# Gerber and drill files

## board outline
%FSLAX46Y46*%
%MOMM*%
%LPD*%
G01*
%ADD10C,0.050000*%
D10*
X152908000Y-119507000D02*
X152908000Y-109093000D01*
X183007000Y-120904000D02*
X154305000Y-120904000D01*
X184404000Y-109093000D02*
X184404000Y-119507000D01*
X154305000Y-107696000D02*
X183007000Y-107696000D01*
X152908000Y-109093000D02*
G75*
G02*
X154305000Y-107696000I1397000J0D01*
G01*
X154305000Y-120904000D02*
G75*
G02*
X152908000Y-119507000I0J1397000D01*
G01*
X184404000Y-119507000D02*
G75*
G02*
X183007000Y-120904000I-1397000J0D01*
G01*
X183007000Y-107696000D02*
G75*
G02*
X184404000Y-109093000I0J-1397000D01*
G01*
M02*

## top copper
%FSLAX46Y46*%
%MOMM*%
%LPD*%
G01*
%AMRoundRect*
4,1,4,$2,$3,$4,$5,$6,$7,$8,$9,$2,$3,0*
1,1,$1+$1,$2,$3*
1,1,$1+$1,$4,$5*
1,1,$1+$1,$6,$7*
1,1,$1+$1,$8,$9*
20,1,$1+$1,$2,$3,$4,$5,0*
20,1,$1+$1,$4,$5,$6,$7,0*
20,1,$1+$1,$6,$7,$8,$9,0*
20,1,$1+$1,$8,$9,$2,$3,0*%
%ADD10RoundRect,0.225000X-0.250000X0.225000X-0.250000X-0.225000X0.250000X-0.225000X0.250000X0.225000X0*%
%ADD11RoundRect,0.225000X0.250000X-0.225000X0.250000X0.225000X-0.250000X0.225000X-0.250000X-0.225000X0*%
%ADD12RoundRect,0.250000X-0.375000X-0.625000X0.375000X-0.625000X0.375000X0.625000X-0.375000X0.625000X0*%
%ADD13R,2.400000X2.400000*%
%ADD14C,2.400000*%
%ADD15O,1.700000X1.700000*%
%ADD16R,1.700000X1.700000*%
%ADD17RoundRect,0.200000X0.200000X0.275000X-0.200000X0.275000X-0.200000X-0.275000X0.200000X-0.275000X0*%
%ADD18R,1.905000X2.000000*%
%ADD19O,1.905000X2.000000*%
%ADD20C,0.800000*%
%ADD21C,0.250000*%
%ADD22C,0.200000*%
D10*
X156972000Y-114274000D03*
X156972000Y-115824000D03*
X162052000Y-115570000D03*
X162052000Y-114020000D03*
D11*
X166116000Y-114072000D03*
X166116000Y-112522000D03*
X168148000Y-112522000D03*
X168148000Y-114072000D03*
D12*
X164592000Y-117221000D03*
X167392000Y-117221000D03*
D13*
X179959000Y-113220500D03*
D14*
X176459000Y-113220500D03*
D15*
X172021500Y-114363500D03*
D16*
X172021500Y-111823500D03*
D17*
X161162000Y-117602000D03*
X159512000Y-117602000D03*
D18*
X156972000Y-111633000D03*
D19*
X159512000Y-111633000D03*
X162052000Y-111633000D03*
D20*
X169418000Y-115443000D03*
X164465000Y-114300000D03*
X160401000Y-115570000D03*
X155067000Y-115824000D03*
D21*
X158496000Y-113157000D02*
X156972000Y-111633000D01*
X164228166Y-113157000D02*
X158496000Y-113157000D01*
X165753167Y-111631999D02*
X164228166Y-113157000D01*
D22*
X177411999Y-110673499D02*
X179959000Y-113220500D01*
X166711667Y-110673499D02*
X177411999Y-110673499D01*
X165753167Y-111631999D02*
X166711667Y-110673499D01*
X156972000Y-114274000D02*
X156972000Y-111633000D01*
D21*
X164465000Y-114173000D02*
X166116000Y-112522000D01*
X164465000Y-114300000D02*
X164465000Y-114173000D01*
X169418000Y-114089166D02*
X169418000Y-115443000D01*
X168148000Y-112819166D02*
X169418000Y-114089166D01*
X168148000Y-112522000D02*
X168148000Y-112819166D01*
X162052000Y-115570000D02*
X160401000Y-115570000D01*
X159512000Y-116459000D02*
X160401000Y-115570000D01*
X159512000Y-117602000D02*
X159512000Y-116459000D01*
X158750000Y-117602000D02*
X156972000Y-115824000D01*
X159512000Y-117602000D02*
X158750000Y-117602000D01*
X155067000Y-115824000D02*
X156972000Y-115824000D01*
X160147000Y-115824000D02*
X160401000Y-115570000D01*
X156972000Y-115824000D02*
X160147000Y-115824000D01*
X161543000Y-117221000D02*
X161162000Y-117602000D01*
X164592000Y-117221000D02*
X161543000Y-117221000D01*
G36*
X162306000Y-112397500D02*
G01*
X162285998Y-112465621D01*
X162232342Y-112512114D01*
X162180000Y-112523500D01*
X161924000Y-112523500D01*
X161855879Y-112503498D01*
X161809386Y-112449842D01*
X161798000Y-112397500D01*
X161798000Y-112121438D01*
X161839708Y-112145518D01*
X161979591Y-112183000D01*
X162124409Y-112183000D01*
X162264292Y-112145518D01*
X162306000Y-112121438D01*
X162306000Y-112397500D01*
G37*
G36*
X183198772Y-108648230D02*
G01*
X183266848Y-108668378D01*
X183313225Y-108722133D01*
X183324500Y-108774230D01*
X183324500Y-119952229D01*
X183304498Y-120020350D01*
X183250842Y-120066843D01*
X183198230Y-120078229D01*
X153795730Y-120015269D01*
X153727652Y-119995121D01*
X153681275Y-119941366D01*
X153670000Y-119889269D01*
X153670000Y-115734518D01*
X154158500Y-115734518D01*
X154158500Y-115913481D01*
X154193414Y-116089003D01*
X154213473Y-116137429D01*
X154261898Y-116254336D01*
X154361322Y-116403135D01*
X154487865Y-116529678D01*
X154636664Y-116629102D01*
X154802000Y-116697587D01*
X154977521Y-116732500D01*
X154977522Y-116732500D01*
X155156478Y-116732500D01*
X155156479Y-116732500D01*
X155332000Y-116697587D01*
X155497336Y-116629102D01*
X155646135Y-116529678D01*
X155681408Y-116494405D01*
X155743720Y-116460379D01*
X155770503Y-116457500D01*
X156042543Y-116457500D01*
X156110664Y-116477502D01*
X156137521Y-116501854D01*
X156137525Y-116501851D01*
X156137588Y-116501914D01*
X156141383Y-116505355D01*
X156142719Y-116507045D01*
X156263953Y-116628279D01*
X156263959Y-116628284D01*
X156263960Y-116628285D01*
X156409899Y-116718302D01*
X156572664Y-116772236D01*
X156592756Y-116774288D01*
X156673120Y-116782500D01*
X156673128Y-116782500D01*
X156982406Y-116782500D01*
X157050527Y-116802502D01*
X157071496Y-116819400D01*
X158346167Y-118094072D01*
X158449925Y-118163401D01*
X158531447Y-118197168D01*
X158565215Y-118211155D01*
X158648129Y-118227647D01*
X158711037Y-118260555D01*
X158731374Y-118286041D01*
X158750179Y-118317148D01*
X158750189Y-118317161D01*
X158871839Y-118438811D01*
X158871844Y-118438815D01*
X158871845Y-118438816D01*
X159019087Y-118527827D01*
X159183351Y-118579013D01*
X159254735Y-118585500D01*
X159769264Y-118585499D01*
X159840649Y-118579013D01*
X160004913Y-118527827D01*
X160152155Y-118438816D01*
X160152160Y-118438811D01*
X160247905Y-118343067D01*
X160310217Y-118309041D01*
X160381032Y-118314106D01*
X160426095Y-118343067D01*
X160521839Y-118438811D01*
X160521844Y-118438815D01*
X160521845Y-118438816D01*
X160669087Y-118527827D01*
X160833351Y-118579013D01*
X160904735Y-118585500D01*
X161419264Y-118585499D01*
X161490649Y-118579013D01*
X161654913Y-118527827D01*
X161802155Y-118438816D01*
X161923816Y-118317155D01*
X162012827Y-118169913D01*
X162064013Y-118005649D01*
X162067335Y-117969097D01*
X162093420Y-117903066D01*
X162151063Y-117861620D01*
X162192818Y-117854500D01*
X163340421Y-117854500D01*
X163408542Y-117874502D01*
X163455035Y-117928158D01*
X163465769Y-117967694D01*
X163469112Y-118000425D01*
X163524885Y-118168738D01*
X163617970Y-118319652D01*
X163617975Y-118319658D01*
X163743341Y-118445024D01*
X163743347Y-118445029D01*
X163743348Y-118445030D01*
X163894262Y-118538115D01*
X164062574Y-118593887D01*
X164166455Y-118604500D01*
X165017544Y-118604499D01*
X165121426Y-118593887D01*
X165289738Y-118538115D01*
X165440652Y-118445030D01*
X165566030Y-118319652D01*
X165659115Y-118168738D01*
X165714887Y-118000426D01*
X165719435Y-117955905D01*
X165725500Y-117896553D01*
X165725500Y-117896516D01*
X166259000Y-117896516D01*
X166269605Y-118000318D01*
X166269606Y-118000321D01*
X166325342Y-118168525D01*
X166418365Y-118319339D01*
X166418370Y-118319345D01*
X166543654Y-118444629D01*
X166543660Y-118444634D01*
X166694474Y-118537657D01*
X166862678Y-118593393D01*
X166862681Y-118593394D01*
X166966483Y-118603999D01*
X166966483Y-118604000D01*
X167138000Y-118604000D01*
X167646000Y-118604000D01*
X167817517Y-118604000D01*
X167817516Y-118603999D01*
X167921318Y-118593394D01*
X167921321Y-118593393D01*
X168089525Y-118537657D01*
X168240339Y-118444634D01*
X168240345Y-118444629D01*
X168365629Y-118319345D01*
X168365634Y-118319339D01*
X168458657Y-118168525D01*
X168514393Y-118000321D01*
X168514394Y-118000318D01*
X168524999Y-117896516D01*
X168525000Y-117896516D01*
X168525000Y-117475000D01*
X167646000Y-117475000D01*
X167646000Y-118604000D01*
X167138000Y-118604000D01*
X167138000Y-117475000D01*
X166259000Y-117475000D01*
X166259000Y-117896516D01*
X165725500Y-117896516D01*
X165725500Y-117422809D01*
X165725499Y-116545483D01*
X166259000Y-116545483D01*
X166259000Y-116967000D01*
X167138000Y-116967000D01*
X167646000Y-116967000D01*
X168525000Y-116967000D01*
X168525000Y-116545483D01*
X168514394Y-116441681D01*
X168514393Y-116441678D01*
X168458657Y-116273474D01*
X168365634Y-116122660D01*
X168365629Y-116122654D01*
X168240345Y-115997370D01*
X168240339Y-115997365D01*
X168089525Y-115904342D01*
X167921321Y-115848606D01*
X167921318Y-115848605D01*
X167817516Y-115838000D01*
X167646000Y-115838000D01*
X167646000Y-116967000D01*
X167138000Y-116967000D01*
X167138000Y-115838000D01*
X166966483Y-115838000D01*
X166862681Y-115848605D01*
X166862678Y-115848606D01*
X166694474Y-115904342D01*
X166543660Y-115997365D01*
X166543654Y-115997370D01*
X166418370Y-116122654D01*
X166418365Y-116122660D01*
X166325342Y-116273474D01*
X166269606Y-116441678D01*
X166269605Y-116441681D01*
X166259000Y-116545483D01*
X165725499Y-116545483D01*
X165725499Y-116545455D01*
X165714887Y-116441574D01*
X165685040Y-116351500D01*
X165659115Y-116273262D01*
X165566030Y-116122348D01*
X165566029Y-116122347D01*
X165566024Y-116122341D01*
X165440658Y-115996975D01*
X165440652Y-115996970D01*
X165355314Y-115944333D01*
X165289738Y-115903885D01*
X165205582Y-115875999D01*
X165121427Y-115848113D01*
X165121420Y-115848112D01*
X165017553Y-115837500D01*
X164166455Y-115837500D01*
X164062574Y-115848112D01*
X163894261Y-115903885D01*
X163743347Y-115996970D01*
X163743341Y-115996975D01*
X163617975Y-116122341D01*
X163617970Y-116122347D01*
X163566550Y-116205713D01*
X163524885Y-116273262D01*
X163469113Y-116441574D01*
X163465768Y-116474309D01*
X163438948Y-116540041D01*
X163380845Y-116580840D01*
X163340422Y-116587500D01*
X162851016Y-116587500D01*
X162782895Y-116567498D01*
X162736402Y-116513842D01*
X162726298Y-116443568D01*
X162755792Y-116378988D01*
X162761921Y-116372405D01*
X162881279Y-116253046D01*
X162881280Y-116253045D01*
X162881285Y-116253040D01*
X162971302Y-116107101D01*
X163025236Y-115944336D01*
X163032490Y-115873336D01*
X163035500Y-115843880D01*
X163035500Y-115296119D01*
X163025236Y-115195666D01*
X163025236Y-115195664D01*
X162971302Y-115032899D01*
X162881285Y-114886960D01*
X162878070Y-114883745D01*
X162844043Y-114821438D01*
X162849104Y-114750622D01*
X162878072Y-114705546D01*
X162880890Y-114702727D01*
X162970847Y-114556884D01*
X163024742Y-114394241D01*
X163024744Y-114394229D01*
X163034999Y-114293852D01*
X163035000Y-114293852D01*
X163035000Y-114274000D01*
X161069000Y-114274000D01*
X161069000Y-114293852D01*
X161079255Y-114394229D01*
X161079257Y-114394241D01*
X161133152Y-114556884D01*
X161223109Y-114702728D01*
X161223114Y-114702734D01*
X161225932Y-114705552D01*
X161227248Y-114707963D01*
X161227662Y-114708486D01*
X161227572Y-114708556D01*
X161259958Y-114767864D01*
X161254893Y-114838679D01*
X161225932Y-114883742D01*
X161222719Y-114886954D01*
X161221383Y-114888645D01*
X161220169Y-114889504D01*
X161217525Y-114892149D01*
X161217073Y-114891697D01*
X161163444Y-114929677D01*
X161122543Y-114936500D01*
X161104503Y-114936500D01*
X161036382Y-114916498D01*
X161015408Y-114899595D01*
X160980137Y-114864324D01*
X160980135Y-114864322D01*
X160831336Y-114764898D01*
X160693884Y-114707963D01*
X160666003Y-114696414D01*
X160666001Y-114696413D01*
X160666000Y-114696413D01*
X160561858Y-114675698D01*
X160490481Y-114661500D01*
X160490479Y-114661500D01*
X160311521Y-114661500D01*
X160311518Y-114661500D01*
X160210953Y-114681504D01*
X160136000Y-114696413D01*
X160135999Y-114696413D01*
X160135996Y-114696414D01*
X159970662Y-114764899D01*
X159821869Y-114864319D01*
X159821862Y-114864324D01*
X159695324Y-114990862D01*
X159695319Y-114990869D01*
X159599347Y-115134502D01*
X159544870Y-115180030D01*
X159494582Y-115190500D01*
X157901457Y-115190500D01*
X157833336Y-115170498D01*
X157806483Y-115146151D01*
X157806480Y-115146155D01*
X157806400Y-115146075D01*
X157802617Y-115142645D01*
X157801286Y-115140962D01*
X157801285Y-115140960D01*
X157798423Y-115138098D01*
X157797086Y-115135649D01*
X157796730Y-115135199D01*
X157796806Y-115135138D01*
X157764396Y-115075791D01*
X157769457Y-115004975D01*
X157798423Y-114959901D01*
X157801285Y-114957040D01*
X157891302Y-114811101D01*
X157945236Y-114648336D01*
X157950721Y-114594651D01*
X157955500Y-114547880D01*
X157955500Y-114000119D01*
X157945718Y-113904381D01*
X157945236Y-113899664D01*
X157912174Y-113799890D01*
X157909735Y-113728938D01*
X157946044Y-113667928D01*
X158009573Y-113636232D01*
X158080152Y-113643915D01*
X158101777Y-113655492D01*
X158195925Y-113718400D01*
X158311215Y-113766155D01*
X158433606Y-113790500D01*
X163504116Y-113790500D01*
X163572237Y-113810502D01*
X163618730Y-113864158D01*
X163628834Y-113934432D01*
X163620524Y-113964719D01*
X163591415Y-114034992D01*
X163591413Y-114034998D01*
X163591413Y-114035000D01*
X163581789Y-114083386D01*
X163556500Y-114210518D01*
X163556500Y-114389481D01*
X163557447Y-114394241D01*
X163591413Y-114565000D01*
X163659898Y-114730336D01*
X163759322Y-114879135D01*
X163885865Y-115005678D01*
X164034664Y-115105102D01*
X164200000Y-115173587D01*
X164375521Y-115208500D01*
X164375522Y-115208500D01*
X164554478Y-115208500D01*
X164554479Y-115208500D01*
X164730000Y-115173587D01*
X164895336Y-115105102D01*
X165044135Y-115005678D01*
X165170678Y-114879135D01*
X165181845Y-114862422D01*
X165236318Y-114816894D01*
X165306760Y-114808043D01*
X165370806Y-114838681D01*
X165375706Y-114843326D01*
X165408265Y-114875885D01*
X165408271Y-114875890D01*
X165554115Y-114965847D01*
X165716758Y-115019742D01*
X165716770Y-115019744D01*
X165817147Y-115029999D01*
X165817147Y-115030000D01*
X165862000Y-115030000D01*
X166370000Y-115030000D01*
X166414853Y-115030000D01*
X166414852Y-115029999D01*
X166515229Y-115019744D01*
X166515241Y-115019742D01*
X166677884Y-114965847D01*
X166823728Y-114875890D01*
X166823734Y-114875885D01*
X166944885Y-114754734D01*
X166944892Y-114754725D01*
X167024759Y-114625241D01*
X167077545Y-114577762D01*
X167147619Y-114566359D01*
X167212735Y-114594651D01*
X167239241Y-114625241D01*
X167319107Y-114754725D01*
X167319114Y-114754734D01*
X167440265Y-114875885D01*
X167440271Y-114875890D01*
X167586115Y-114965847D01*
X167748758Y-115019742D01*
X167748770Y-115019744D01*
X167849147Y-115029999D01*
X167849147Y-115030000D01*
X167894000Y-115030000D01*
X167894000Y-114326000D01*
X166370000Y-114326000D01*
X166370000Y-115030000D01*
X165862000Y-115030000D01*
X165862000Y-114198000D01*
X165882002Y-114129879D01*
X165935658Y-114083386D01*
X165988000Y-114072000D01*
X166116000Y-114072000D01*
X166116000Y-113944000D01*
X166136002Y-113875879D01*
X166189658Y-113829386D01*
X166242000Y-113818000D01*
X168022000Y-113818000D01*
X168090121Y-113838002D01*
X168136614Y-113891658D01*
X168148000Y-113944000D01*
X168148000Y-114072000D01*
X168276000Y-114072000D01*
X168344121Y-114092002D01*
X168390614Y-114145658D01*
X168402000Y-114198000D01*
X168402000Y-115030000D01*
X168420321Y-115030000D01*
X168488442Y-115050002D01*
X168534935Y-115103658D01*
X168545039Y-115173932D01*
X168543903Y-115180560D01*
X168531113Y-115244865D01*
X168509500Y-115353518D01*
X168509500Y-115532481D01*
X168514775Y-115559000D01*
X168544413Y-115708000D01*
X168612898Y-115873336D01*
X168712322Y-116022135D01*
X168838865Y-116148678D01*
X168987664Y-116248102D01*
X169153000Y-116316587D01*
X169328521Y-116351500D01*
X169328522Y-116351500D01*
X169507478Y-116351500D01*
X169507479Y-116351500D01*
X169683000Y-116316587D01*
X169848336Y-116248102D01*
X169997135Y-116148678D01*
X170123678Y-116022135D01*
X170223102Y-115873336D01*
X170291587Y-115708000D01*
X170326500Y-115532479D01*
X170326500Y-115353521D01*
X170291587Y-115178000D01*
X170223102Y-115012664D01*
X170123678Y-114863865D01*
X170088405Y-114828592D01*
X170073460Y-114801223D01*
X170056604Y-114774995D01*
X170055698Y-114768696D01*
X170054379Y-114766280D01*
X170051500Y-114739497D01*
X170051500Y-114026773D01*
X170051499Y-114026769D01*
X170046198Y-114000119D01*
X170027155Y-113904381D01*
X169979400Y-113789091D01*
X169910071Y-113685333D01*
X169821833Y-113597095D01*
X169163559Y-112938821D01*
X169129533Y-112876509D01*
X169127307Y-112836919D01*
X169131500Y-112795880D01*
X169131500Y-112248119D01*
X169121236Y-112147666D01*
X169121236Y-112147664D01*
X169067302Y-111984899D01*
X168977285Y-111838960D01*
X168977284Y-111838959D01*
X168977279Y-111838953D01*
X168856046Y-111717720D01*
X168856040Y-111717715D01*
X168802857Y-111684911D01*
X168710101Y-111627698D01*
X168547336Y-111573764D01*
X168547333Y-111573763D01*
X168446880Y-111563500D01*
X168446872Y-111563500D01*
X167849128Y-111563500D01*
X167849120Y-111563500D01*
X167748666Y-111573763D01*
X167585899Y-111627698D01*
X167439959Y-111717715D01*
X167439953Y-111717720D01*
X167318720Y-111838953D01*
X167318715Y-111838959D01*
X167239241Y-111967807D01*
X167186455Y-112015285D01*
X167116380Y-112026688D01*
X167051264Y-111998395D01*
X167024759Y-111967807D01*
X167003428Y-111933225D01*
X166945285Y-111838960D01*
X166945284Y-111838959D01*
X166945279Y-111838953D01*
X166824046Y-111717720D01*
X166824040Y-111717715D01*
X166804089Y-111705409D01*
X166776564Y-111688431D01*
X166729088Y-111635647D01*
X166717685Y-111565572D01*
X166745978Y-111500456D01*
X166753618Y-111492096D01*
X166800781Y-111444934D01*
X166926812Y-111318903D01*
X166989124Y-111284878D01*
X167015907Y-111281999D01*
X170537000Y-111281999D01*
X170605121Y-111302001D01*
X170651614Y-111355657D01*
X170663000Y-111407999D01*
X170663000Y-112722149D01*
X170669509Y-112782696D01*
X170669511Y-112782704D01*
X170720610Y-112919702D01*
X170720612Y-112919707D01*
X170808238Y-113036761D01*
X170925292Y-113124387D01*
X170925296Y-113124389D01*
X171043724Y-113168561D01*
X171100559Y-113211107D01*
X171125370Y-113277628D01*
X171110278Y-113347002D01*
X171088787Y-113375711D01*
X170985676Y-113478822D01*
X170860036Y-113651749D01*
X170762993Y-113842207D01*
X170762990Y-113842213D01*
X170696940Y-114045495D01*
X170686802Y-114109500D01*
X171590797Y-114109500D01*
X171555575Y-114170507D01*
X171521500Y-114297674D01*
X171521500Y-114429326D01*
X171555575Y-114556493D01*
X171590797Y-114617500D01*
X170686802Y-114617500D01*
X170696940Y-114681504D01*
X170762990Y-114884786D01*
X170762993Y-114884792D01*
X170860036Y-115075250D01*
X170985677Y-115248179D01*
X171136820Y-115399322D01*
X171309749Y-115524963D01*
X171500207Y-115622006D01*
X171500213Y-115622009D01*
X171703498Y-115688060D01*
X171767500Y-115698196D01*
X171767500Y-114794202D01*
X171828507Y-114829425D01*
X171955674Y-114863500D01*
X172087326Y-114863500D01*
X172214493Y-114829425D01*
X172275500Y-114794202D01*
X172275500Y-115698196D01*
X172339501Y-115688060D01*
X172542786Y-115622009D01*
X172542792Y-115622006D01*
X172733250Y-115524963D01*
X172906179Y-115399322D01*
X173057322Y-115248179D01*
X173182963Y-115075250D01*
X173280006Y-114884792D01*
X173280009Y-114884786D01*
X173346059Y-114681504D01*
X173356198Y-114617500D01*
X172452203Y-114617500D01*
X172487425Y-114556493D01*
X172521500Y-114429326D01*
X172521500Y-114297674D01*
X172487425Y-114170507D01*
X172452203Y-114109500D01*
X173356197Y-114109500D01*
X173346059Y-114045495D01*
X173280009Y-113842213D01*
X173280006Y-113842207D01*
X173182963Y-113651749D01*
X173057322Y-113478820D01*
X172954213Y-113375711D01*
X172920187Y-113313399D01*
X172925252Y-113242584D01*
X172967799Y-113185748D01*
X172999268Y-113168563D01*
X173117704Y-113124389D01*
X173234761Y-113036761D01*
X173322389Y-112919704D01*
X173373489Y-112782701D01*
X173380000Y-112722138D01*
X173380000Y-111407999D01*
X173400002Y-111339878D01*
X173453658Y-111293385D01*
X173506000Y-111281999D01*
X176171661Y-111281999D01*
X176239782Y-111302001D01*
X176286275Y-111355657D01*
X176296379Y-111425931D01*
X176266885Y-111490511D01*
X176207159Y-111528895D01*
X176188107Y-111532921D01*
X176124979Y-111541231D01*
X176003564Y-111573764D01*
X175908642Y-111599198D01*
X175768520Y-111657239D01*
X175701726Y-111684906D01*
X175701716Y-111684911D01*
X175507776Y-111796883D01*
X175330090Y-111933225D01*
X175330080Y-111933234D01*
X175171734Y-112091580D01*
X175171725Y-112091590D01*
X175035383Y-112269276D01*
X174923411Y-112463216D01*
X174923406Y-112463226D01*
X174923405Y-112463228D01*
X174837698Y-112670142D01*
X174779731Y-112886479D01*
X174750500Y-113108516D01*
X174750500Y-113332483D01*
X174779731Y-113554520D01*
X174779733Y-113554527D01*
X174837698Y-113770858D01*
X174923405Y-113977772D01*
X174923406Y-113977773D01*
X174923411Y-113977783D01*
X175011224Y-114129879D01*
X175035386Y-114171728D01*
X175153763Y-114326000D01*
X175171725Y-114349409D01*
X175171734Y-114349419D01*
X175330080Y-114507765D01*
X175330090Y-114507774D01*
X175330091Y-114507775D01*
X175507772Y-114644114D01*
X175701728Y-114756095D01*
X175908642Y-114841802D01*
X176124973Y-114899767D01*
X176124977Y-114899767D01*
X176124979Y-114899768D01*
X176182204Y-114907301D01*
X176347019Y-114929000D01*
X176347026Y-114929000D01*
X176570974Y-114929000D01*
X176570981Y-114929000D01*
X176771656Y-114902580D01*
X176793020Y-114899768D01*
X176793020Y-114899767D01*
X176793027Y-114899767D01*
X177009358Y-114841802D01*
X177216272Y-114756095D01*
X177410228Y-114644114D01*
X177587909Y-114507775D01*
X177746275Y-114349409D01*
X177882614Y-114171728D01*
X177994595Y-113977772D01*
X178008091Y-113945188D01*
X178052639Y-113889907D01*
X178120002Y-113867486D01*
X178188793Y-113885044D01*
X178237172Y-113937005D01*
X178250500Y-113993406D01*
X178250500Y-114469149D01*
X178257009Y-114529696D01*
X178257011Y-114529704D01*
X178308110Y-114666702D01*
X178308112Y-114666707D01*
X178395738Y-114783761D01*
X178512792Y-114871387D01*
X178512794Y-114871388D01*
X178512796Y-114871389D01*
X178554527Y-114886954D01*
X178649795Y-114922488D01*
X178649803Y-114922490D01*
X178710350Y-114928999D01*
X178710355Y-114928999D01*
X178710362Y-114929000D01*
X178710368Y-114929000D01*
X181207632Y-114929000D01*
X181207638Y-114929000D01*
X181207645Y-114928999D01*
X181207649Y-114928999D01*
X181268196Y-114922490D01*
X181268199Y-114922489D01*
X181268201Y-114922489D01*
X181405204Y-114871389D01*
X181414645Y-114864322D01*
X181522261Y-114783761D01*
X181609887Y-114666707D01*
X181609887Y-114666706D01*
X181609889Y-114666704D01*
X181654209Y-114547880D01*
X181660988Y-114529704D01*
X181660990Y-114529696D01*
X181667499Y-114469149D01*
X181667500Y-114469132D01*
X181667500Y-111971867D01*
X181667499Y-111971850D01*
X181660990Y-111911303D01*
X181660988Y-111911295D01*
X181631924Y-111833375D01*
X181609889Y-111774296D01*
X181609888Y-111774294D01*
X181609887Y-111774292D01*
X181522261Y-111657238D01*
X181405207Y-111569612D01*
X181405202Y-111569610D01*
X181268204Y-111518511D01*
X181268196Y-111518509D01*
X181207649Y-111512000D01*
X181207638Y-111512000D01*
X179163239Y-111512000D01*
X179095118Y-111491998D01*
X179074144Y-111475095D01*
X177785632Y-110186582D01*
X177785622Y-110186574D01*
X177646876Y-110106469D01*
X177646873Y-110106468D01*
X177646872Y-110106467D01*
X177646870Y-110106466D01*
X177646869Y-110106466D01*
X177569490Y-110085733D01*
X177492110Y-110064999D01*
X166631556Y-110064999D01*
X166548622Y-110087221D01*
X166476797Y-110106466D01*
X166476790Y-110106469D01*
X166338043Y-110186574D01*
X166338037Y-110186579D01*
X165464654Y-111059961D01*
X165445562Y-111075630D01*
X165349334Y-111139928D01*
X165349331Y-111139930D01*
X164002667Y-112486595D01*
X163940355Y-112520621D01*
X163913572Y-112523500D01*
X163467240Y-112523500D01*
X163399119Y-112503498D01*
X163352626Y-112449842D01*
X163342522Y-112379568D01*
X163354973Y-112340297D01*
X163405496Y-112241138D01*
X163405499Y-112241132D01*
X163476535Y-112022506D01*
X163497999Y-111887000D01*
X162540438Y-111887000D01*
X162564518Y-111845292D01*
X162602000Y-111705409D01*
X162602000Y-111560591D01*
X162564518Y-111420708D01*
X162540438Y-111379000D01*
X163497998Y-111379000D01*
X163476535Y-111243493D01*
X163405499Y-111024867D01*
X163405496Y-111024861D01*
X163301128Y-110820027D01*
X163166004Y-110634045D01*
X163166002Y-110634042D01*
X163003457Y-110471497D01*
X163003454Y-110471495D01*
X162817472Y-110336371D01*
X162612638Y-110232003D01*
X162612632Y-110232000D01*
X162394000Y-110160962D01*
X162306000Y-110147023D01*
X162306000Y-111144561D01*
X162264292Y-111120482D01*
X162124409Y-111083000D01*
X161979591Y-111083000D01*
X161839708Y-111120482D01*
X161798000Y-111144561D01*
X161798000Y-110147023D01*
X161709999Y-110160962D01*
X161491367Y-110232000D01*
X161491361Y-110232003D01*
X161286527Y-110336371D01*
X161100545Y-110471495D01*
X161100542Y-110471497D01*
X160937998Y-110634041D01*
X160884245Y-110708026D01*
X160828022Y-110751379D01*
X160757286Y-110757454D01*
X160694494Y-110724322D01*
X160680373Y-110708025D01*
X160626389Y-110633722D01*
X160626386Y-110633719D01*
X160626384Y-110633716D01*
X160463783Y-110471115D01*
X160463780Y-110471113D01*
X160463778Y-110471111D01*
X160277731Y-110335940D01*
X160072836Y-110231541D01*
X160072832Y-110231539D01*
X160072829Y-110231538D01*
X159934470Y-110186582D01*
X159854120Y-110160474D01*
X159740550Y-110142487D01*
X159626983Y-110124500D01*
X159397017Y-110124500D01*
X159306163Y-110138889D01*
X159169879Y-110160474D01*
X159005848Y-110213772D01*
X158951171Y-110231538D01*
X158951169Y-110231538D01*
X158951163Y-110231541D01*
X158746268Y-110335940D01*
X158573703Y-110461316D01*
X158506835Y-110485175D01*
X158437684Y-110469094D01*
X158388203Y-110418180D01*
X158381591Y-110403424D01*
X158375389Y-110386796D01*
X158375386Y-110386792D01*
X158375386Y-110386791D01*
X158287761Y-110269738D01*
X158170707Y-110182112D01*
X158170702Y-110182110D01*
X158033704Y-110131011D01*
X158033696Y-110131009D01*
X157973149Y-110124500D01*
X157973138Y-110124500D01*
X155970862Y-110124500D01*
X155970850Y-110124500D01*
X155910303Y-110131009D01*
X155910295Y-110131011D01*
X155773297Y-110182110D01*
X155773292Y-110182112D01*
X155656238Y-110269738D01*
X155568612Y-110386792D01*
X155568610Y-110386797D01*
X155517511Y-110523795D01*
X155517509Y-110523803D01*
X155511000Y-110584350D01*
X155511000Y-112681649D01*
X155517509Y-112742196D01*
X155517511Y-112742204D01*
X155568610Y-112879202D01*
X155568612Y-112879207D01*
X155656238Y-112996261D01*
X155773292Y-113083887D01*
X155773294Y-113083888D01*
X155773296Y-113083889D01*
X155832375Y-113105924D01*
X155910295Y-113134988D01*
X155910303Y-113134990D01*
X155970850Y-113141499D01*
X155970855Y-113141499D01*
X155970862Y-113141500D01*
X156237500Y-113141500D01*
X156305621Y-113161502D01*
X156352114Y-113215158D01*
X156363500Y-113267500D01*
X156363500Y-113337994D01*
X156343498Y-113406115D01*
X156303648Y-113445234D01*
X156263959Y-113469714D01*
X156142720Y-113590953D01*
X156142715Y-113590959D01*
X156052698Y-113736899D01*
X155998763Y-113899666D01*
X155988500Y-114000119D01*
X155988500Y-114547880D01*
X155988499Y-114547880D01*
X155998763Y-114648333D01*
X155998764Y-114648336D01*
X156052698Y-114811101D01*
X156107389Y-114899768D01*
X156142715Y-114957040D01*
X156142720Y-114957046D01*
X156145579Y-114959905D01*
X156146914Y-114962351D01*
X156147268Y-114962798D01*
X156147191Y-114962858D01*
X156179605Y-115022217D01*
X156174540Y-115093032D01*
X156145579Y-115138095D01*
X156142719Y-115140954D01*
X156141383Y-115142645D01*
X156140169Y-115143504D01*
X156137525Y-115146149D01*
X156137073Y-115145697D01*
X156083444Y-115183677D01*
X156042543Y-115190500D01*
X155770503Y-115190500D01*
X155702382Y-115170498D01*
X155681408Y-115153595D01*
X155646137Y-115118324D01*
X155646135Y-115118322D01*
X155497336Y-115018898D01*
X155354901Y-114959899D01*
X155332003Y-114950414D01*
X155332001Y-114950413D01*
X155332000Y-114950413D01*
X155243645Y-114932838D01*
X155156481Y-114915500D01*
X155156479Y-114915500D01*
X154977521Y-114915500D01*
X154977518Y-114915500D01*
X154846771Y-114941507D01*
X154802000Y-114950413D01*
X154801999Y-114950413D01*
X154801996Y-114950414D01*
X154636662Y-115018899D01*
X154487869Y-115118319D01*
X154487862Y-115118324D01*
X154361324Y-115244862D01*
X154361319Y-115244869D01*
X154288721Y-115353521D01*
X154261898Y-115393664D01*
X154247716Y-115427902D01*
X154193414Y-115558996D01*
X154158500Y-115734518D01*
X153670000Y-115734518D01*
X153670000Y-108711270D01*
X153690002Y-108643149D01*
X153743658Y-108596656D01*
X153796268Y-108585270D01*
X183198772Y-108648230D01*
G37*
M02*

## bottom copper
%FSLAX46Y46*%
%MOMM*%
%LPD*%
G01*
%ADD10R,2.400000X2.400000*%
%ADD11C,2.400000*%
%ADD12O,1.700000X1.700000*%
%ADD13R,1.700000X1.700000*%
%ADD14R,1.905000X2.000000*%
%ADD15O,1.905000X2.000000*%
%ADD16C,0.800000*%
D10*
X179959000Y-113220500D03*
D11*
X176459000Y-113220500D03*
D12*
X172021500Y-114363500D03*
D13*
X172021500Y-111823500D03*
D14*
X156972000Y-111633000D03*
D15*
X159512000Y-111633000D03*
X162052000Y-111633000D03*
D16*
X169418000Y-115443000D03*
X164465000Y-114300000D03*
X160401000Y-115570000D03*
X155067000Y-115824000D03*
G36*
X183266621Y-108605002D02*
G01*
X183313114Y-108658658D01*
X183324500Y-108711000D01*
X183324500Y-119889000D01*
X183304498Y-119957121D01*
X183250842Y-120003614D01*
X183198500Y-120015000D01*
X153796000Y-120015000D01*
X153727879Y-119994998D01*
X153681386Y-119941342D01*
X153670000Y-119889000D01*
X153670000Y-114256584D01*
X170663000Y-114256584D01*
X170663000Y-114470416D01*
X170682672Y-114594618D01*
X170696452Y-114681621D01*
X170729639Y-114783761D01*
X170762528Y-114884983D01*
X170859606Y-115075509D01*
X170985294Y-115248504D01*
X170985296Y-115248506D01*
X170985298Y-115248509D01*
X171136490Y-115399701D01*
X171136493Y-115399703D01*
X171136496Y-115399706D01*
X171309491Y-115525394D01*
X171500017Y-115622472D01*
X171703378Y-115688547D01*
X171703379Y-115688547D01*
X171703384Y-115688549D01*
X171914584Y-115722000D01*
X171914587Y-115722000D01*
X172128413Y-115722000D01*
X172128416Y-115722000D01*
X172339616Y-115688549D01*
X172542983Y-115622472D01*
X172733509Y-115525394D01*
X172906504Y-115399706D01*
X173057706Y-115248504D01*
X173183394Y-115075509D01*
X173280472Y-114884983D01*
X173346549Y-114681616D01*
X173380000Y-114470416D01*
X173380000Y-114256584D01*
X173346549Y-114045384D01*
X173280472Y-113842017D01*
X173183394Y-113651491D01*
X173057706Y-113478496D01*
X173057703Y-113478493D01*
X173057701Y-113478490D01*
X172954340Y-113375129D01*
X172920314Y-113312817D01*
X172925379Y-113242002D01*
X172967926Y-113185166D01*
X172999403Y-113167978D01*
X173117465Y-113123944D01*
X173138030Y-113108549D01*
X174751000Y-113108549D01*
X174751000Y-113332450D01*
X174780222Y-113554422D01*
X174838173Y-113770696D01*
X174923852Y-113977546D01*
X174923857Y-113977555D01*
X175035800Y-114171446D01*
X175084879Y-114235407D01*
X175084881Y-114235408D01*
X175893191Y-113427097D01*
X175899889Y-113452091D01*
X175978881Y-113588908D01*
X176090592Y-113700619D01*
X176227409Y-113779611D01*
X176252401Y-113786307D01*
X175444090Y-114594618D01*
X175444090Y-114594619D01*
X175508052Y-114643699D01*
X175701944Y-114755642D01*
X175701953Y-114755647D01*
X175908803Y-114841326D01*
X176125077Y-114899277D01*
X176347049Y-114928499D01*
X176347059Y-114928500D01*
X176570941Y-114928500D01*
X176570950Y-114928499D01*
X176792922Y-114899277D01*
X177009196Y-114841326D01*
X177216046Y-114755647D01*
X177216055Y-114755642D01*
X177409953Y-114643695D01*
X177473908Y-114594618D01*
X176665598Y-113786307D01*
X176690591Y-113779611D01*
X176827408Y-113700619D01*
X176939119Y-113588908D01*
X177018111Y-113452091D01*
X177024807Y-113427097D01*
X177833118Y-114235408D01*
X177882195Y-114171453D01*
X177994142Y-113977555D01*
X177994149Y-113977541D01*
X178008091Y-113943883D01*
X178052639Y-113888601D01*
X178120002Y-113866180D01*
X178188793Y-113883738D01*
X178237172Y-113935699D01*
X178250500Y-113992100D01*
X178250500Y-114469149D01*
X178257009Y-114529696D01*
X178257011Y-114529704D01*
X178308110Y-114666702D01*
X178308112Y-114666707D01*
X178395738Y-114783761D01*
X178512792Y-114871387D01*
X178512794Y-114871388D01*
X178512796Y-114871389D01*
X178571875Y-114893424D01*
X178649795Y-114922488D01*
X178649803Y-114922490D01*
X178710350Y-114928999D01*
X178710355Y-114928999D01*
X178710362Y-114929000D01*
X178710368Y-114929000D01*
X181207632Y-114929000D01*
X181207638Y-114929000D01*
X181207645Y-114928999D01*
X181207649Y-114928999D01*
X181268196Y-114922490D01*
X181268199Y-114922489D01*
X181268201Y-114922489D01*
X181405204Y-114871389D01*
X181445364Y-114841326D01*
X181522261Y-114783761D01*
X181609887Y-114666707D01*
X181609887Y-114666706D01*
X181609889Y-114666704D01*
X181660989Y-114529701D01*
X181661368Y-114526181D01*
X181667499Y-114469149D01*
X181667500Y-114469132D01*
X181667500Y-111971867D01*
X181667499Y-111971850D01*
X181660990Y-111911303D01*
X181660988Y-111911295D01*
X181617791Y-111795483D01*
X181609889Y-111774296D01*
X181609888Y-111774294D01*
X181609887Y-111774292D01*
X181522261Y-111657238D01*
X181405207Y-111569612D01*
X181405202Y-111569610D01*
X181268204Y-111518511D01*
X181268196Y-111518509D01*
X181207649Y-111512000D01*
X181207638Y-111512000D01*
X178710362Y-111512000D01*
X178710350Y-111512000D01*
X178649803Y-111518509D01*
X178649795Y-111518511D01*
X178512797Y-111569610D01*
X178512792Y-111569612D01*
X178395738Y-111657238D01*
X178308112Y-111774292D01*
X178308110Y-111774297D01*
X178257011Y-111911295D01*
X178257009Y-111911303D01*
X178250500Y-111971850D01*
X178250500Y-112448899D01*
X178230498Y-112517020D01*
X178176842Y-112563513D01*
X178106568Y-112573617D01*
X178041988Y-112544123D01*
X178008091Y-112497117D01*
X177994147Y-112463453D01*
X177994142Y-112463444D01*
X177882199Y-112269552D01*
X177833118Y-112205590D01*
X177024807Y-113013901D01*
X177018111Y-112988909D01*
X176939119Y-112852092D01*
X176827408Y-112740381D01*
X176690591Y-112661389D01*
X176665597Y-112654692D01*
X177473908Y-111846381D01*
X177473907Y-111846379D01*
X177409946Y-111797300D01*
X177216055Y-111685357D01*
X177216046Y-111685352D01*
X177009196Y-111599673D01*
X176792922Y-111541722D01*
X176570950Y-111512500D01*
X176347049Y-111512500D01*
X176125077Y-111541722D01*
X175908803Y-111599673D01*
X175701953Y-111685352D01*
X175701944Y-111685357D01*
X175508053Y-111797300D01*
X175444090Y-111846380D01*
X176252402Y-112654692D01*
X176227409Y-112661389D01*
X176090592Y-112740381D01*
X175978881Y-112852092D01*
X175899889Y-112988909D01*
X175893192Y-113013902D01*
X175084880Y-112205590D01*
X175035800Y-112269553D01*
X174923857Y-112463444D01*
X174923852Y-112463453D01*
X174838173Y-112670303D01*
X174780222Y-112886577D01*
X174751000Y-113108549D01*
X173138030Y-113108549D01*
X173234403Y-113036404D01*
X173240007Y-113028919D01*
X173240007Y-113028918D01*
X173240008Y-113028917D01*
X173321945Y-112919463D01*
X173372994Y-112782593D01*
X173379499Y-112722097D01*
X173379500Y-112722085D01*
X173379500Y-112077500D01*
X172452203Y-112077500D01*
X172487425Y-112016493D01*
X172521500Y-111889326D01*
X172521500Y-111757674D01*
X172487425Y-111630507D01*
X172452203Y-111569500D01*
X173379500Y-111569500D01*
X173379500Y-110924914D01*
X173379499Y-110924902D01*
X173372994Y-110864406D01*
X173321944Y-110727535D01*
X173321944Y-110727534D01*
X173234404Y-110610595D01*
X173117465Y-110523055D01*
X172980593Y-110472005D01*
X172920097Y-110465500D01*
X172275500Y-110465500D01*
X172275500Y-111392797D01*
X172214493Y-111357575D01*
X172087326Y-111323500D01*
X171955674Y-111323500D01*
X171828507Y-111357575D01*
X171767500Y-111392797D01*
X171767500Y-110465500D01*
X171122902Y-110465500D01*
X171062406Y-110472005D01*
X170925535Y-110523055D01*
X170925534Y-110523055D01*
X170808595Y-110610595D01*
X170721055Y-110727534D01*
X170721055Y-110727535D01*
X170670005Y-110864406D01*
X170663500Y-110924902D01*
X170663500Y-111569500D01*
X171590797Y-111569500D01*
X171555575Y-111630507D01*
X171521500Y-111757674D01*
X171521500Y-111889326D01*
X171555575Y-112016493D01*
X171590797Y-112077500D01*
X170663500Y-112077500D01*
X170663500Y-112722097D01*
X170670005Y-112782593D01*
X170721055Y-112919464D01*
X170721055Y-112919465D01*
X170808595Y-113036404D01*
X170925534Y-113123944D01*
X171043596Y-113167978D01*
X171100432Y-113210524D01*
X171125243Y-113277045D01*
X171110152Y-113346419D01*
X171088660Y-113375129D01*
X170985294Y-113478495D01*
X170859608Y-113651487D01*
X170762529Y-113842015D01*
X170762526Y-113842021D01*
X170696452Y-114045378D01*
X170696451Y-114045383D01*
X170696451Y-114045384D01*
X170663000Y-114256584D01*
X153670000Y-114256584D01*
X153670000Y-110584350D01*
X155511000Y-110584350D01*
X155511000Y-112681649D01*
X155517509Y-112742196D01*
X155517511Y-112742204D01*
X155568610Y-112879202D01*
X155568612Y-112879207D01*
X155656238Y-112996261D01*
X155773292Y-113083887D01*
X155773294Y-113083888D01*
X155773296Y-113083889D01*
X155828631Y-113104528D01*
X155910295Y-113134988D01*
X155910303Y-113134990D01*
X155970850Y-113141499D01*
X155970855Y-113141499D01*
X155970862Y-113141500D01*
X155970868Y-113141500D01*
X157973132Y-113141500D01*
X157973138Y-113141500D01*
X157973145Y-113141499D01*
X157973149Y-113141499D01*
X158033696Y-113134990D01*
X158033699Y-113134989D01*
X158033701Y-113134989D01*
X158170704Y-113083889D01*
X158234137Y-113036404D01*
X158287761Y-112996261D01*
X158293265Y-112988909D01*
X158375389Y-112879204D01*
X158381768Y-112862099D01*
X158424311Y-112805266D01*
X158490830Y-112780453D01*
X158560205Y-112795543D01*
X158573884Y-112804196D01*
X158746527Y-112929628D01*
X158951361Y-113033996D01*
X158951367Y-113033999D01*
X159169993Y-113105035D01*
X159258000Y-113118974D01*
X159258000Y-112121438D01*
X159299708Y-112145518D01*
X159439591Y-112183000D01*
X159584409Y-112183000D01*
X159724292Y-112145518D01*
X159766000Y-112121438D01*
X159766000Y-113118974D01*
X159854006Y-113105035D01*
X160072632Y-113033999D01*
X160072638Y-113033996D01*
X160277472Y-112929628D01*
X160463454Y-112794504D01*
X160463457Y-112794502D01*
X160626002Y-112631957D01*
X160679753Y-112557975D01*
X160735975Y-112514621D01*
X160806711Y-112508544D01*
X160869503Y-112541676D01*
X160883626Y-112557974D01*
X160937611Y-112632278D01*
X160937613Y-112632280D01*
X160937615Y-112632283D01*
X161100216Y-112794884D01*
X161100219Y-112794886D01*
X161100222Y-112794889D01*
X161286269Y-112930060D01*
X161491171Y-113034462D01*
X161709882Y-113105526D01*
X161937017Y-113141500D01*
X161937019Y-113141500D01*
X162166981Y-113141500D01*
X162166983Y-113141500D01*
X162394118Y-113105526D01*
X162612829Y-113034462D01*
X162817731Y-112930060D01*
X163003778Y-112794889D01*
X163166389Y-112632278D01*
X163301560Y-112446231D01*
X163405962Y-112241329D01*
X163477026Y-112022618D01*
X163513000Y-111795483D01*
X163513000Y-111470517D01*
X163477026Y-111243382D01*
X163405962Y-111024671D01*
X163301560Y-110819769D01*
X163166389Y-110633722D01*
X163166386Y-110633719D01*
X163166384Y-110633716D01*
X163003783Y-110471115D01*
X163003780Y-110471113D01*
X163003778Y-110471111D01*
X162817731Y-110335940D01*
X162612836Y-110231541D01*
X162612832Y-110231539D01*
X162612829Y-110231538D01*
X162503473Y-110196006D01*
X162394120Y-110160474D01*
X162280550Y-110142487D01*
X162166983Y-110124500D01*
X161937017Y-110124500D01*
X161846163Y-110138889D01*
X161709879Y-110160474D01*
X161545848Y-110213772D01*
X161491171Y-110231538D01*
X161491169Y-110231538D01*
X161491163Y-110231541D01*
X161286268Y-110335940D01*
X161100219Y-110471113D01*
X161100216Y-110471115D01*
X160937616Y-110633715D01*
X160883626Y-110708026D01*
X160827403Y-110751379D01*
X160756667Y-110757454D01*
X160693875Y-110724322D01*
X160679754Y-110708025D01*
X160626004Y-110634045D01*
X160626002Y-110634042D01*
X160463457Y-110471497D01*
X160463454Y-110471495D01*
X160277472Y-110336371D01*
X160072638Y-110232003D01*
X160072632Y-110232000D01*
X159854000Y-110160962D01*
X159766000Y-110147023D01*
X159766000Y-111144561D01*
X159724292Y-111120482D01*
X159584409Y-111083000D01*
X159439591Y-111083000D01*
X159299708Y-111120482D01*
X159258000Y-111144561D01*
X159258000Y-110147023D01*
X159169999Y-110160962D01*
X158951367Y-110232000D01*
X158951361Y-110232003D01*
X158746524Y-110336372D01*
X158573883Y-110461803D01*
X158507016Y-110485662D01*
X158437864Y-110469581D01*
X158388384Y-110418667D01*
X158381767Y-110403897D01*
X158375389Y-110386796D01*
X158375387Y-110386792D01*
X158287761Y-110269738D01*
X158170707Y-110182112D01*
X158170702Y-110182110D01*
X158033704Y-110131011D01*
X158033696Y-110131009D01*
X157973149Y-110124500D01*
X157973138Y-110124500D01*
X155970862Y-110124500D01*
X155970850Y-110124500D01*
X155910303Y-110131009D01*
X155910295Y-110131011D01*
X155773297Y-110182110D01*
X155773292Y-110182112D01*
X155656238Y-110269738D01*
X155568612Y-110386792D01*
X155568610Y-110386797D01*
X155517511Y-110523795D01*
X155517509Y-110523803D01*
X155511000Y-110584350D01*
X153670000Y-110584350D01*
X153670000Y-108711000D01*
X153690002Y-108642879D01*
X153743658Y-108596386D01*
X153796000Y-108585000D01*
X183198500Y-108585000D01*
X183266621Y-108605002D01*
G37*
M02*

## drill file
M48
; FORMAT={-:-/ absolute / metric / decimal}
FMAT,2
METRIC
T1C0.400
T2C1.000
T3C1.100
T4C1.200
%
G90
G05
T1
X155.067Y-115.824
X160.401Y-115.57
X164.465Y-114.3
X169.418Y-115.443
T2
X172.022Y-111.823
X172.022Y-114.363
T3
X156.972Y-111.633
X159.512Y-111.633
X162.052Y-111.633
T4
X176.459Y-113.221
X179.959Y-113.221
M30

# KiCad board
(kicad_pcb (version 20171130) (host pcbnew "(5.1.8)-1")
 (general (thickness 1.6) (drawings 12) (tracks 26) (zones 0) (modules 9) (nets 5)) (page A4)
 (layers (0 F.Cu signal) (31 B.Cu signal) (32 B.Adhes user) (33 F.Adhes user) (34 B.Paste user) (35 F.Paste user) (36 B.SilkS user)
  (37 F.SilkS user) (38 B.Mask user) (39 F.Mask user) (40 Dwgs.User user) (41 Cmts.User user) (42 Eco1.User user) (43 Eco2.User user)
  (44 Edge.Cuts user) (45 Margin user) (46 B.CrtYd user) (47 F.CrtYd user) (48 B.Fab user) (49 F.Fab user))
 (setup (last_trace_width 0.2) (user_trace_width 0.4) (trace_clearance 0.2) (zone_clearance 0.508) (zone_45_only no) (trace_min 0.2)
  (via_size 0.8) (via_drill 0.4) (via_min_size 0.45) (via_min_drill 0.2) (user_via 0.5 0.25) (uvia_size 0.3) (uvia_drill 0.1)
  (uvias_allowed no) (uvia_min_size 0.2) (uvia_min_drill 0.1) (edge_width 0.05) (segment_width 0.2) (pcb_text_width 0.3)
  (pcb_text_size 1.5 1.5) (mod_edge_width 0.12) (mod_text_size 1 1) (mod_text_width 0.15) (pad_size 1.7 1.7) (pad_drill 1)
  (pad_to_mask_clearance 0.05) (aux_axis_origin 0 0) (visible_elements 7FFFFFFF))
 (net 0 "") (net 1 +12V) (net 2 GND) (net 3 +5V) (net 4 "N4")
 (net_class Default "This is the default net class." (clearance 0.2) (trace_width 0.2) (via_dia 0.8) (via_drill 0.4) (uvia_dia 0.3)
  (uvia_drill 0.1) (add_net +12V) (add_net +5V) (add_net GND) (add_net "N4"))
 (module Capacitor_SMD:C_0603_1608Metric (layer F.Cu) (at 156.972 115.049 270)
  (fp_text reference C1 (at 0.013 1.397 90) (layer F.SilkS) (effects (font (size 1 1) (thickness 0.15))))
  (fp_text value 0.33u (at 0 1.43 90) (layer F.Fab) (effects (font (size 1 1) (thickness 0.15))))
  (pad 1 smd roundrect (at -0.775 0 270) (size 0.9 0.95) (layers F.Cu F.Paste F.Mask) (roundrect_rratio 0.25) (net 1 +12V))
  (pad 2 smd roundrect (at 0.775 0 270) (size 0.9 0.95) (layers F.Cu F.Paste F.Mask) (roundrect_rratio 0.25) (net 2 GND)))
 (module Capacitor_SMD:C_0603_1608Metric (layer F.Cu) (at 162.052 114.795 270)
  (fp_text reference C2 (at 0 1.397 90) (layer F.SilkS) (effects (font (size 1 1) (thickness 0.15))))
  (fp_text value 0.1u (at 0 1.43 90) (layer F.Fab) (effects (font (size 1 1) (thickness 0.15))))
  (pad 2 smd roundrect (at 0.775 0 270) (size 0.9 0.95) (layers F.Cu F.Paste F.Mask) (roundrect_rratio 0.25) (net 2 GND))
  (pad 1 smd roundrect (at -0.775 0 270) (size 0.9 0.95) (layers F.Cu F.Paste F.Mask) (roundrect_rratio 0.25) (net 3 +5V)))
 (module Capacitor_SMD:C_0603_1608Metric (layer F.Cu) (at 166.116 113.297 90)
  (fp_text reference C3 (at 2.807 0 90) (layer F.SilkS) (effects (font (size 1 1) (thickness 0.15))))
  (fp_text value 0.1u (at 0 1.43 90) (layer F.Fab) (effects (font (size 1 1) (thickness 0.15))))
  (pad 1 smd roundrect (at -0.775 0 90) (size 0.9 0.95) (layers F.Cu F.Paste F.Mask) (roundrect_rratio 0.25) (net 3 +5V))
  (pad 2 smd roundrect (at 0.775 0 90) (size 0.9 0.95) (layers F.Cu F.Paste F.Mask) (roundrect_rratio 0.25) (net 2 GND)))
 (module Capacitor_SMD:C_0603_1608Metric (layer F.Cu) (at 168.148 113.297 90)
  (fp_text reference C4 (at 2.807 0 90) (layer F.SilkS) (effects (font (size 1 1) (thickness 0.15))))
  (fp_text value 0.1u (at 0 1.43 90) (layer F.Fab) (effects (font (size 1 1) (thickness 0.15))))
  (pad 2 smd roundrect (at 0.775 0 90) (size 0.9 0.95) (layers F.Cu F.Paste F.Mask) (roundrect_rratio 0.25) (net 2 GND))
  (pad 1 smd roundrect (at -0.775 0 90) (size 0.9 0.95) (layers F.Cu F.Paste F.Mask) (roundrect_rratio 0.25) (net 3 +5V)))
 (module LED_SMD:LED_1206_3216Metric (layer F.Cu) (at 165.992 117.221)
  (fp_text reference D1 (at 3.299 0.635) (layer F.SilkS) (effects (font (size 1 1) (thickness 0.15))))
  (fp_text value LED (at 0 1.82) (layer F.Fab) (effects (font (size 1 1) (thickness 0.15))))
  (pad 1 smd roundrect (at -1.4 0) (size 1.25 1.75) (layers F.Cu F.Paste F.Mask) (roundrect_rratio 0.2) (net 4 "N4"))
  (pad 2 smd roundrect (at 1.4 0) (size 1.25 1.75) (layers F.Cu F.Paste F.Mask) (roundrect_rratio 0.2) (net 3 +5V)))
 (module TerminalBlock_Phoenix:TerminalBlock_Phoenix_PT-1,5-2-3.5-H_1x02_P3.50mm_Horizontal (layer F.Cu) (at 179.959 113.2205 180)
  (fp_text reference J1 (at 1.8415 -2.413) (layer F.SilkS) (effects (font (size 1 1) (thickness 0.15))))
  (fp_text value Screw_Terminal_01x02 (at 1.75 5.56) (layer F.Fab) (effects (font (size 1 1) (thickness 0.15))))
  (pad 1 thru_hole rect (at 0 0 180) (size 2.4 2.4) (drill 1.2) (layers *.Cu *.Mask) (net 1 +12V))
  (pad 2 thru_hole circle (at 3.5 0 180) (size 2.4 2.4) (drill 1.2) (layers *.Cu *.Mask) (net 2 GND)))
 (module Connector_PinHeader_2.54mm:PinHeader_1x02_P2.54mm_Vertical (layer F.Cu) (at 172.0215 111.8235)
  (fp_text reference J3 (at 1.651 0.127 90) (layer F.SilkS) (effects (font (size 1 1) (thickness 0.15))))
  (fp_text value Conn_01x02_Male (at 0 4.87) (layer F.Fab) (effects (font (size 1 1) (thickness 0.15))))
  (pad 2 thru_hole oval (at 0 2.54) (size 1.7 1.7) (drill 1) (layers *.Cu *.Mask) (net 3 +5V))
  (pad 1 thru_hole rect (at 0 0) (size 1.7 1.7) (drill 1) (layers *.Cu *.Mask) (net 2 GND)))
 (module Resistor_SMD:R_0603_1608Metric (layer F.Cu) (at 160.337 117.602 180)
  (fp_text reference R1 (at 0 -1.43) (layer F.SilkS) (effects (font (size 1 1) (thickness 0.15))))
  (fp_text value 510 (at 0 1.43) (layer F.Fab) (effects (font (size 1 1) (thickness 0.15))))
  (pad 1 smd roundrect (at -0.825 0 180) (size 0.8 0.95) (layers F.Cu F.Paste F.Mask) (roundrect_rratio 0.25) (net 4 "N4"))
  (pad 2 smd roundrect (at 0.825 0 180) (size 0.8 0.95) (layers F.Cu F.Paste F.Mask) (roundrect_rratio 0.25) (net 2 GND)))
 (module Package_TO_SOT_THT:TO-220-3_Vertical (layer F.Cu) (at 156.972 111.633)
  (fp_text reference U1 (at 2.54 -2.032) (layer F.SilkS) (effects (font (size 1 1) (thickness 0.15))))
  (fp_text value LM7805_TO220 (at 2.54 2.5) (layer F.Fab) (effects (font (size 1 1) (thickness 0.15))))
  (pad 1 thru_hole rect (at 0 0) (size 1.905 2) (drill 1.1) (layers *.Cu *.Mask) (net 1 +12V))
  (pad 2 thru_hole oval (at 2.54 0) (size 1.905 2) (drill 1.1) (layers *.Cu *.Mask) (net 2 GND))
  (pad 3 thru_hole oval (at 5.08 0) (size 1.905 2) (drill 1.1) (layers *.Cu *.Mask) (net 3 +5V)))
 (gr_line (start 152.908 119.507) (end 152.908 109.093) (layer Edge.Cuts) (width 0.05))
 (gr_line (start 183.007 120.904) (end 154.305 120.904) (layer Edge.Cuts) (width 0.05))
 (gr_line (start 184.404 109.093) (end 184.404 119.507) (layer Edge.Cuts) (width 0.05))
 (gr_line (start 154.305 107.696) (end 183.007 107.696) (layer Edge.Cuts) (width 0.05))
 (gr_arc (start 154.305 109.093) (end 154.305 107.696) (angle -90) (layer Edge.Cuts) (width 0.05))
 (gr_arc (start 154.305 119.507) (end 152.908 119.507) (angle -90) (layer Edge.Cuts) (width 0.05))
 (gr_arc (start 183.007 119.507) (end 183.007 120.904) (angle -90) (layer Edge.Cuts) (width 0.05))
 (gr_arc (start 183.007 109.093) (end 184.404 109.093) (angle -90) (layer Edge.Cuts) (width 0.05))
 (segment (start 158.496 113.157) (end 156.972 111.633) (width 0.25) (layer F.Cu) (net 1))
 (segment (start 164.228166 113.157) (end 158.496 113.157) (width 0.25) (layer F.Cu) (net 1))
 (segment (start 165.753167 111.631999) (end 164.228166 113.157) (width 0.25) (layer F.Cu) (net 1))
 (segment (start 177.411999 110.673499) (end 179.959 113.2205) (width 0.2) (layer F.Cu) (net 1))
 (segment (start 166.711667 110.673499) (end 177.411999 110.673499) (width 0.2) (layer F.Cu) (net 1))
 (segment (start 165.753167 111.631999) (end 166.711667 110.673499) (width 0.2) (layer F.Cu) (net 1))
 (segment (start 156.972 114.274) (end 156.972 111.633) (width 0.2) (layer F.Cu) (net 1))
 (via (at 169.418 115.443) (size 0.8) (drill 0.4) (layers F.Cu B.Cu) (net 2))
 (via (at 164.465 114.3) (size 0.8) (drill 0.4) (layers F.Cu B.Cu) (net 2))
 (via (at 160.401 115.57) (size 0.8) (drill 0.4) (layers F.Cu B.Cu) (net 2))
 (via (at 155.067 115.824) (size 0.8) (drill 0.4) (layers F.Cu B.Cu) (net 2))
 (segment (start 164.465 114.173) (end 166.116 112.522) (width 0.25) (layer F.Cu) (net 2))
 (segment (start 164.465 114.3) (end 164.465 114.173) (width 0.25) (layer F.Cu) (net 2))
 (segment (start 169.418 114.089166) (end 169.418 115.443) (width 0.25) (layer F.Cu) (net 2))
 (segment (start 168.148 112.819166) (end 169.418 114.089166) (width 0.25) (layer F.Cu) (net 2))
 (segment (start 168.148 112.522) (end 168.148 112.819166) (width 0.25) (layer F.Cu) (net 2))
 (segment (start 162.052 115.57) (end 160.401 115.57) (width 0.25) (layer F.Cu) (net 2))
 (segment (start 159.512 116.459) (end 160.401 115.57) (width 0.25) (layer F.Cu) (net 2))
 (segment (start 159.512 117.602) (end 159.512 116.459) (width 0.25) (layer F.Cu) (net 2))
 (segment (start 158.75 117.602) (end 156.972 115.824) (width 0.25) (layer F.Cu) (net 2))
 (segment (start 159.512 117.602) (end 158.75 117.602) (width 0.25) (layer F.Cu) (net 2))
 (segment (start 155.067 115.824) (end 156.972 115.824) (width 0.25) (layer F.Cu) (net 2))
 (segment (start 160.147 115.824) (end 160.401 115.57) (width 0.25) (layer F.Cu) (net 2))
 (segment (start 156.972 115.824) (end 160.147 115.824) (width 0.25) (layer F.Cu) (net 2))
 (segment (start 161.543 117.221) (end 161.162 117.602) (width 0.25) (layer F.Cu) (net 4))
 (segment (start 164.592 117.221) (end 161.543 117.221) (width 0.25) (layer F.Cu) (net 4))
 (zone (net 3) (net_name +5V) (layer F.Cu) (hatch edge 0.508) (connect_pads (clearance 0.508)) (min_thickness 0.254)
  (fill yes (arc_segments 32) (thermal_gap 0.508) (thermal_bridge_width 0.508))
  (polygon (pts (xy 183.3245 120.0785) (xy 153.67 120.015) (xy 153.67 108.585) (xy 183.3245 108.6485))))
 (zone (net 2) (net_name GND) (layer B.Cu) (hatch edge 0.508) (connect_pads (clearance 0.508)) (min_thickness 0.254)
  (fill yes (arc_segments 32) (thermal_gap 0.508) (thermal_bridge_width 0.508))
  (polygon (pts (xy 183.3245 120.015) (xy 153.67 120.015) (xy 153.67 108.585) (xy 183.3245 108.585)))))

